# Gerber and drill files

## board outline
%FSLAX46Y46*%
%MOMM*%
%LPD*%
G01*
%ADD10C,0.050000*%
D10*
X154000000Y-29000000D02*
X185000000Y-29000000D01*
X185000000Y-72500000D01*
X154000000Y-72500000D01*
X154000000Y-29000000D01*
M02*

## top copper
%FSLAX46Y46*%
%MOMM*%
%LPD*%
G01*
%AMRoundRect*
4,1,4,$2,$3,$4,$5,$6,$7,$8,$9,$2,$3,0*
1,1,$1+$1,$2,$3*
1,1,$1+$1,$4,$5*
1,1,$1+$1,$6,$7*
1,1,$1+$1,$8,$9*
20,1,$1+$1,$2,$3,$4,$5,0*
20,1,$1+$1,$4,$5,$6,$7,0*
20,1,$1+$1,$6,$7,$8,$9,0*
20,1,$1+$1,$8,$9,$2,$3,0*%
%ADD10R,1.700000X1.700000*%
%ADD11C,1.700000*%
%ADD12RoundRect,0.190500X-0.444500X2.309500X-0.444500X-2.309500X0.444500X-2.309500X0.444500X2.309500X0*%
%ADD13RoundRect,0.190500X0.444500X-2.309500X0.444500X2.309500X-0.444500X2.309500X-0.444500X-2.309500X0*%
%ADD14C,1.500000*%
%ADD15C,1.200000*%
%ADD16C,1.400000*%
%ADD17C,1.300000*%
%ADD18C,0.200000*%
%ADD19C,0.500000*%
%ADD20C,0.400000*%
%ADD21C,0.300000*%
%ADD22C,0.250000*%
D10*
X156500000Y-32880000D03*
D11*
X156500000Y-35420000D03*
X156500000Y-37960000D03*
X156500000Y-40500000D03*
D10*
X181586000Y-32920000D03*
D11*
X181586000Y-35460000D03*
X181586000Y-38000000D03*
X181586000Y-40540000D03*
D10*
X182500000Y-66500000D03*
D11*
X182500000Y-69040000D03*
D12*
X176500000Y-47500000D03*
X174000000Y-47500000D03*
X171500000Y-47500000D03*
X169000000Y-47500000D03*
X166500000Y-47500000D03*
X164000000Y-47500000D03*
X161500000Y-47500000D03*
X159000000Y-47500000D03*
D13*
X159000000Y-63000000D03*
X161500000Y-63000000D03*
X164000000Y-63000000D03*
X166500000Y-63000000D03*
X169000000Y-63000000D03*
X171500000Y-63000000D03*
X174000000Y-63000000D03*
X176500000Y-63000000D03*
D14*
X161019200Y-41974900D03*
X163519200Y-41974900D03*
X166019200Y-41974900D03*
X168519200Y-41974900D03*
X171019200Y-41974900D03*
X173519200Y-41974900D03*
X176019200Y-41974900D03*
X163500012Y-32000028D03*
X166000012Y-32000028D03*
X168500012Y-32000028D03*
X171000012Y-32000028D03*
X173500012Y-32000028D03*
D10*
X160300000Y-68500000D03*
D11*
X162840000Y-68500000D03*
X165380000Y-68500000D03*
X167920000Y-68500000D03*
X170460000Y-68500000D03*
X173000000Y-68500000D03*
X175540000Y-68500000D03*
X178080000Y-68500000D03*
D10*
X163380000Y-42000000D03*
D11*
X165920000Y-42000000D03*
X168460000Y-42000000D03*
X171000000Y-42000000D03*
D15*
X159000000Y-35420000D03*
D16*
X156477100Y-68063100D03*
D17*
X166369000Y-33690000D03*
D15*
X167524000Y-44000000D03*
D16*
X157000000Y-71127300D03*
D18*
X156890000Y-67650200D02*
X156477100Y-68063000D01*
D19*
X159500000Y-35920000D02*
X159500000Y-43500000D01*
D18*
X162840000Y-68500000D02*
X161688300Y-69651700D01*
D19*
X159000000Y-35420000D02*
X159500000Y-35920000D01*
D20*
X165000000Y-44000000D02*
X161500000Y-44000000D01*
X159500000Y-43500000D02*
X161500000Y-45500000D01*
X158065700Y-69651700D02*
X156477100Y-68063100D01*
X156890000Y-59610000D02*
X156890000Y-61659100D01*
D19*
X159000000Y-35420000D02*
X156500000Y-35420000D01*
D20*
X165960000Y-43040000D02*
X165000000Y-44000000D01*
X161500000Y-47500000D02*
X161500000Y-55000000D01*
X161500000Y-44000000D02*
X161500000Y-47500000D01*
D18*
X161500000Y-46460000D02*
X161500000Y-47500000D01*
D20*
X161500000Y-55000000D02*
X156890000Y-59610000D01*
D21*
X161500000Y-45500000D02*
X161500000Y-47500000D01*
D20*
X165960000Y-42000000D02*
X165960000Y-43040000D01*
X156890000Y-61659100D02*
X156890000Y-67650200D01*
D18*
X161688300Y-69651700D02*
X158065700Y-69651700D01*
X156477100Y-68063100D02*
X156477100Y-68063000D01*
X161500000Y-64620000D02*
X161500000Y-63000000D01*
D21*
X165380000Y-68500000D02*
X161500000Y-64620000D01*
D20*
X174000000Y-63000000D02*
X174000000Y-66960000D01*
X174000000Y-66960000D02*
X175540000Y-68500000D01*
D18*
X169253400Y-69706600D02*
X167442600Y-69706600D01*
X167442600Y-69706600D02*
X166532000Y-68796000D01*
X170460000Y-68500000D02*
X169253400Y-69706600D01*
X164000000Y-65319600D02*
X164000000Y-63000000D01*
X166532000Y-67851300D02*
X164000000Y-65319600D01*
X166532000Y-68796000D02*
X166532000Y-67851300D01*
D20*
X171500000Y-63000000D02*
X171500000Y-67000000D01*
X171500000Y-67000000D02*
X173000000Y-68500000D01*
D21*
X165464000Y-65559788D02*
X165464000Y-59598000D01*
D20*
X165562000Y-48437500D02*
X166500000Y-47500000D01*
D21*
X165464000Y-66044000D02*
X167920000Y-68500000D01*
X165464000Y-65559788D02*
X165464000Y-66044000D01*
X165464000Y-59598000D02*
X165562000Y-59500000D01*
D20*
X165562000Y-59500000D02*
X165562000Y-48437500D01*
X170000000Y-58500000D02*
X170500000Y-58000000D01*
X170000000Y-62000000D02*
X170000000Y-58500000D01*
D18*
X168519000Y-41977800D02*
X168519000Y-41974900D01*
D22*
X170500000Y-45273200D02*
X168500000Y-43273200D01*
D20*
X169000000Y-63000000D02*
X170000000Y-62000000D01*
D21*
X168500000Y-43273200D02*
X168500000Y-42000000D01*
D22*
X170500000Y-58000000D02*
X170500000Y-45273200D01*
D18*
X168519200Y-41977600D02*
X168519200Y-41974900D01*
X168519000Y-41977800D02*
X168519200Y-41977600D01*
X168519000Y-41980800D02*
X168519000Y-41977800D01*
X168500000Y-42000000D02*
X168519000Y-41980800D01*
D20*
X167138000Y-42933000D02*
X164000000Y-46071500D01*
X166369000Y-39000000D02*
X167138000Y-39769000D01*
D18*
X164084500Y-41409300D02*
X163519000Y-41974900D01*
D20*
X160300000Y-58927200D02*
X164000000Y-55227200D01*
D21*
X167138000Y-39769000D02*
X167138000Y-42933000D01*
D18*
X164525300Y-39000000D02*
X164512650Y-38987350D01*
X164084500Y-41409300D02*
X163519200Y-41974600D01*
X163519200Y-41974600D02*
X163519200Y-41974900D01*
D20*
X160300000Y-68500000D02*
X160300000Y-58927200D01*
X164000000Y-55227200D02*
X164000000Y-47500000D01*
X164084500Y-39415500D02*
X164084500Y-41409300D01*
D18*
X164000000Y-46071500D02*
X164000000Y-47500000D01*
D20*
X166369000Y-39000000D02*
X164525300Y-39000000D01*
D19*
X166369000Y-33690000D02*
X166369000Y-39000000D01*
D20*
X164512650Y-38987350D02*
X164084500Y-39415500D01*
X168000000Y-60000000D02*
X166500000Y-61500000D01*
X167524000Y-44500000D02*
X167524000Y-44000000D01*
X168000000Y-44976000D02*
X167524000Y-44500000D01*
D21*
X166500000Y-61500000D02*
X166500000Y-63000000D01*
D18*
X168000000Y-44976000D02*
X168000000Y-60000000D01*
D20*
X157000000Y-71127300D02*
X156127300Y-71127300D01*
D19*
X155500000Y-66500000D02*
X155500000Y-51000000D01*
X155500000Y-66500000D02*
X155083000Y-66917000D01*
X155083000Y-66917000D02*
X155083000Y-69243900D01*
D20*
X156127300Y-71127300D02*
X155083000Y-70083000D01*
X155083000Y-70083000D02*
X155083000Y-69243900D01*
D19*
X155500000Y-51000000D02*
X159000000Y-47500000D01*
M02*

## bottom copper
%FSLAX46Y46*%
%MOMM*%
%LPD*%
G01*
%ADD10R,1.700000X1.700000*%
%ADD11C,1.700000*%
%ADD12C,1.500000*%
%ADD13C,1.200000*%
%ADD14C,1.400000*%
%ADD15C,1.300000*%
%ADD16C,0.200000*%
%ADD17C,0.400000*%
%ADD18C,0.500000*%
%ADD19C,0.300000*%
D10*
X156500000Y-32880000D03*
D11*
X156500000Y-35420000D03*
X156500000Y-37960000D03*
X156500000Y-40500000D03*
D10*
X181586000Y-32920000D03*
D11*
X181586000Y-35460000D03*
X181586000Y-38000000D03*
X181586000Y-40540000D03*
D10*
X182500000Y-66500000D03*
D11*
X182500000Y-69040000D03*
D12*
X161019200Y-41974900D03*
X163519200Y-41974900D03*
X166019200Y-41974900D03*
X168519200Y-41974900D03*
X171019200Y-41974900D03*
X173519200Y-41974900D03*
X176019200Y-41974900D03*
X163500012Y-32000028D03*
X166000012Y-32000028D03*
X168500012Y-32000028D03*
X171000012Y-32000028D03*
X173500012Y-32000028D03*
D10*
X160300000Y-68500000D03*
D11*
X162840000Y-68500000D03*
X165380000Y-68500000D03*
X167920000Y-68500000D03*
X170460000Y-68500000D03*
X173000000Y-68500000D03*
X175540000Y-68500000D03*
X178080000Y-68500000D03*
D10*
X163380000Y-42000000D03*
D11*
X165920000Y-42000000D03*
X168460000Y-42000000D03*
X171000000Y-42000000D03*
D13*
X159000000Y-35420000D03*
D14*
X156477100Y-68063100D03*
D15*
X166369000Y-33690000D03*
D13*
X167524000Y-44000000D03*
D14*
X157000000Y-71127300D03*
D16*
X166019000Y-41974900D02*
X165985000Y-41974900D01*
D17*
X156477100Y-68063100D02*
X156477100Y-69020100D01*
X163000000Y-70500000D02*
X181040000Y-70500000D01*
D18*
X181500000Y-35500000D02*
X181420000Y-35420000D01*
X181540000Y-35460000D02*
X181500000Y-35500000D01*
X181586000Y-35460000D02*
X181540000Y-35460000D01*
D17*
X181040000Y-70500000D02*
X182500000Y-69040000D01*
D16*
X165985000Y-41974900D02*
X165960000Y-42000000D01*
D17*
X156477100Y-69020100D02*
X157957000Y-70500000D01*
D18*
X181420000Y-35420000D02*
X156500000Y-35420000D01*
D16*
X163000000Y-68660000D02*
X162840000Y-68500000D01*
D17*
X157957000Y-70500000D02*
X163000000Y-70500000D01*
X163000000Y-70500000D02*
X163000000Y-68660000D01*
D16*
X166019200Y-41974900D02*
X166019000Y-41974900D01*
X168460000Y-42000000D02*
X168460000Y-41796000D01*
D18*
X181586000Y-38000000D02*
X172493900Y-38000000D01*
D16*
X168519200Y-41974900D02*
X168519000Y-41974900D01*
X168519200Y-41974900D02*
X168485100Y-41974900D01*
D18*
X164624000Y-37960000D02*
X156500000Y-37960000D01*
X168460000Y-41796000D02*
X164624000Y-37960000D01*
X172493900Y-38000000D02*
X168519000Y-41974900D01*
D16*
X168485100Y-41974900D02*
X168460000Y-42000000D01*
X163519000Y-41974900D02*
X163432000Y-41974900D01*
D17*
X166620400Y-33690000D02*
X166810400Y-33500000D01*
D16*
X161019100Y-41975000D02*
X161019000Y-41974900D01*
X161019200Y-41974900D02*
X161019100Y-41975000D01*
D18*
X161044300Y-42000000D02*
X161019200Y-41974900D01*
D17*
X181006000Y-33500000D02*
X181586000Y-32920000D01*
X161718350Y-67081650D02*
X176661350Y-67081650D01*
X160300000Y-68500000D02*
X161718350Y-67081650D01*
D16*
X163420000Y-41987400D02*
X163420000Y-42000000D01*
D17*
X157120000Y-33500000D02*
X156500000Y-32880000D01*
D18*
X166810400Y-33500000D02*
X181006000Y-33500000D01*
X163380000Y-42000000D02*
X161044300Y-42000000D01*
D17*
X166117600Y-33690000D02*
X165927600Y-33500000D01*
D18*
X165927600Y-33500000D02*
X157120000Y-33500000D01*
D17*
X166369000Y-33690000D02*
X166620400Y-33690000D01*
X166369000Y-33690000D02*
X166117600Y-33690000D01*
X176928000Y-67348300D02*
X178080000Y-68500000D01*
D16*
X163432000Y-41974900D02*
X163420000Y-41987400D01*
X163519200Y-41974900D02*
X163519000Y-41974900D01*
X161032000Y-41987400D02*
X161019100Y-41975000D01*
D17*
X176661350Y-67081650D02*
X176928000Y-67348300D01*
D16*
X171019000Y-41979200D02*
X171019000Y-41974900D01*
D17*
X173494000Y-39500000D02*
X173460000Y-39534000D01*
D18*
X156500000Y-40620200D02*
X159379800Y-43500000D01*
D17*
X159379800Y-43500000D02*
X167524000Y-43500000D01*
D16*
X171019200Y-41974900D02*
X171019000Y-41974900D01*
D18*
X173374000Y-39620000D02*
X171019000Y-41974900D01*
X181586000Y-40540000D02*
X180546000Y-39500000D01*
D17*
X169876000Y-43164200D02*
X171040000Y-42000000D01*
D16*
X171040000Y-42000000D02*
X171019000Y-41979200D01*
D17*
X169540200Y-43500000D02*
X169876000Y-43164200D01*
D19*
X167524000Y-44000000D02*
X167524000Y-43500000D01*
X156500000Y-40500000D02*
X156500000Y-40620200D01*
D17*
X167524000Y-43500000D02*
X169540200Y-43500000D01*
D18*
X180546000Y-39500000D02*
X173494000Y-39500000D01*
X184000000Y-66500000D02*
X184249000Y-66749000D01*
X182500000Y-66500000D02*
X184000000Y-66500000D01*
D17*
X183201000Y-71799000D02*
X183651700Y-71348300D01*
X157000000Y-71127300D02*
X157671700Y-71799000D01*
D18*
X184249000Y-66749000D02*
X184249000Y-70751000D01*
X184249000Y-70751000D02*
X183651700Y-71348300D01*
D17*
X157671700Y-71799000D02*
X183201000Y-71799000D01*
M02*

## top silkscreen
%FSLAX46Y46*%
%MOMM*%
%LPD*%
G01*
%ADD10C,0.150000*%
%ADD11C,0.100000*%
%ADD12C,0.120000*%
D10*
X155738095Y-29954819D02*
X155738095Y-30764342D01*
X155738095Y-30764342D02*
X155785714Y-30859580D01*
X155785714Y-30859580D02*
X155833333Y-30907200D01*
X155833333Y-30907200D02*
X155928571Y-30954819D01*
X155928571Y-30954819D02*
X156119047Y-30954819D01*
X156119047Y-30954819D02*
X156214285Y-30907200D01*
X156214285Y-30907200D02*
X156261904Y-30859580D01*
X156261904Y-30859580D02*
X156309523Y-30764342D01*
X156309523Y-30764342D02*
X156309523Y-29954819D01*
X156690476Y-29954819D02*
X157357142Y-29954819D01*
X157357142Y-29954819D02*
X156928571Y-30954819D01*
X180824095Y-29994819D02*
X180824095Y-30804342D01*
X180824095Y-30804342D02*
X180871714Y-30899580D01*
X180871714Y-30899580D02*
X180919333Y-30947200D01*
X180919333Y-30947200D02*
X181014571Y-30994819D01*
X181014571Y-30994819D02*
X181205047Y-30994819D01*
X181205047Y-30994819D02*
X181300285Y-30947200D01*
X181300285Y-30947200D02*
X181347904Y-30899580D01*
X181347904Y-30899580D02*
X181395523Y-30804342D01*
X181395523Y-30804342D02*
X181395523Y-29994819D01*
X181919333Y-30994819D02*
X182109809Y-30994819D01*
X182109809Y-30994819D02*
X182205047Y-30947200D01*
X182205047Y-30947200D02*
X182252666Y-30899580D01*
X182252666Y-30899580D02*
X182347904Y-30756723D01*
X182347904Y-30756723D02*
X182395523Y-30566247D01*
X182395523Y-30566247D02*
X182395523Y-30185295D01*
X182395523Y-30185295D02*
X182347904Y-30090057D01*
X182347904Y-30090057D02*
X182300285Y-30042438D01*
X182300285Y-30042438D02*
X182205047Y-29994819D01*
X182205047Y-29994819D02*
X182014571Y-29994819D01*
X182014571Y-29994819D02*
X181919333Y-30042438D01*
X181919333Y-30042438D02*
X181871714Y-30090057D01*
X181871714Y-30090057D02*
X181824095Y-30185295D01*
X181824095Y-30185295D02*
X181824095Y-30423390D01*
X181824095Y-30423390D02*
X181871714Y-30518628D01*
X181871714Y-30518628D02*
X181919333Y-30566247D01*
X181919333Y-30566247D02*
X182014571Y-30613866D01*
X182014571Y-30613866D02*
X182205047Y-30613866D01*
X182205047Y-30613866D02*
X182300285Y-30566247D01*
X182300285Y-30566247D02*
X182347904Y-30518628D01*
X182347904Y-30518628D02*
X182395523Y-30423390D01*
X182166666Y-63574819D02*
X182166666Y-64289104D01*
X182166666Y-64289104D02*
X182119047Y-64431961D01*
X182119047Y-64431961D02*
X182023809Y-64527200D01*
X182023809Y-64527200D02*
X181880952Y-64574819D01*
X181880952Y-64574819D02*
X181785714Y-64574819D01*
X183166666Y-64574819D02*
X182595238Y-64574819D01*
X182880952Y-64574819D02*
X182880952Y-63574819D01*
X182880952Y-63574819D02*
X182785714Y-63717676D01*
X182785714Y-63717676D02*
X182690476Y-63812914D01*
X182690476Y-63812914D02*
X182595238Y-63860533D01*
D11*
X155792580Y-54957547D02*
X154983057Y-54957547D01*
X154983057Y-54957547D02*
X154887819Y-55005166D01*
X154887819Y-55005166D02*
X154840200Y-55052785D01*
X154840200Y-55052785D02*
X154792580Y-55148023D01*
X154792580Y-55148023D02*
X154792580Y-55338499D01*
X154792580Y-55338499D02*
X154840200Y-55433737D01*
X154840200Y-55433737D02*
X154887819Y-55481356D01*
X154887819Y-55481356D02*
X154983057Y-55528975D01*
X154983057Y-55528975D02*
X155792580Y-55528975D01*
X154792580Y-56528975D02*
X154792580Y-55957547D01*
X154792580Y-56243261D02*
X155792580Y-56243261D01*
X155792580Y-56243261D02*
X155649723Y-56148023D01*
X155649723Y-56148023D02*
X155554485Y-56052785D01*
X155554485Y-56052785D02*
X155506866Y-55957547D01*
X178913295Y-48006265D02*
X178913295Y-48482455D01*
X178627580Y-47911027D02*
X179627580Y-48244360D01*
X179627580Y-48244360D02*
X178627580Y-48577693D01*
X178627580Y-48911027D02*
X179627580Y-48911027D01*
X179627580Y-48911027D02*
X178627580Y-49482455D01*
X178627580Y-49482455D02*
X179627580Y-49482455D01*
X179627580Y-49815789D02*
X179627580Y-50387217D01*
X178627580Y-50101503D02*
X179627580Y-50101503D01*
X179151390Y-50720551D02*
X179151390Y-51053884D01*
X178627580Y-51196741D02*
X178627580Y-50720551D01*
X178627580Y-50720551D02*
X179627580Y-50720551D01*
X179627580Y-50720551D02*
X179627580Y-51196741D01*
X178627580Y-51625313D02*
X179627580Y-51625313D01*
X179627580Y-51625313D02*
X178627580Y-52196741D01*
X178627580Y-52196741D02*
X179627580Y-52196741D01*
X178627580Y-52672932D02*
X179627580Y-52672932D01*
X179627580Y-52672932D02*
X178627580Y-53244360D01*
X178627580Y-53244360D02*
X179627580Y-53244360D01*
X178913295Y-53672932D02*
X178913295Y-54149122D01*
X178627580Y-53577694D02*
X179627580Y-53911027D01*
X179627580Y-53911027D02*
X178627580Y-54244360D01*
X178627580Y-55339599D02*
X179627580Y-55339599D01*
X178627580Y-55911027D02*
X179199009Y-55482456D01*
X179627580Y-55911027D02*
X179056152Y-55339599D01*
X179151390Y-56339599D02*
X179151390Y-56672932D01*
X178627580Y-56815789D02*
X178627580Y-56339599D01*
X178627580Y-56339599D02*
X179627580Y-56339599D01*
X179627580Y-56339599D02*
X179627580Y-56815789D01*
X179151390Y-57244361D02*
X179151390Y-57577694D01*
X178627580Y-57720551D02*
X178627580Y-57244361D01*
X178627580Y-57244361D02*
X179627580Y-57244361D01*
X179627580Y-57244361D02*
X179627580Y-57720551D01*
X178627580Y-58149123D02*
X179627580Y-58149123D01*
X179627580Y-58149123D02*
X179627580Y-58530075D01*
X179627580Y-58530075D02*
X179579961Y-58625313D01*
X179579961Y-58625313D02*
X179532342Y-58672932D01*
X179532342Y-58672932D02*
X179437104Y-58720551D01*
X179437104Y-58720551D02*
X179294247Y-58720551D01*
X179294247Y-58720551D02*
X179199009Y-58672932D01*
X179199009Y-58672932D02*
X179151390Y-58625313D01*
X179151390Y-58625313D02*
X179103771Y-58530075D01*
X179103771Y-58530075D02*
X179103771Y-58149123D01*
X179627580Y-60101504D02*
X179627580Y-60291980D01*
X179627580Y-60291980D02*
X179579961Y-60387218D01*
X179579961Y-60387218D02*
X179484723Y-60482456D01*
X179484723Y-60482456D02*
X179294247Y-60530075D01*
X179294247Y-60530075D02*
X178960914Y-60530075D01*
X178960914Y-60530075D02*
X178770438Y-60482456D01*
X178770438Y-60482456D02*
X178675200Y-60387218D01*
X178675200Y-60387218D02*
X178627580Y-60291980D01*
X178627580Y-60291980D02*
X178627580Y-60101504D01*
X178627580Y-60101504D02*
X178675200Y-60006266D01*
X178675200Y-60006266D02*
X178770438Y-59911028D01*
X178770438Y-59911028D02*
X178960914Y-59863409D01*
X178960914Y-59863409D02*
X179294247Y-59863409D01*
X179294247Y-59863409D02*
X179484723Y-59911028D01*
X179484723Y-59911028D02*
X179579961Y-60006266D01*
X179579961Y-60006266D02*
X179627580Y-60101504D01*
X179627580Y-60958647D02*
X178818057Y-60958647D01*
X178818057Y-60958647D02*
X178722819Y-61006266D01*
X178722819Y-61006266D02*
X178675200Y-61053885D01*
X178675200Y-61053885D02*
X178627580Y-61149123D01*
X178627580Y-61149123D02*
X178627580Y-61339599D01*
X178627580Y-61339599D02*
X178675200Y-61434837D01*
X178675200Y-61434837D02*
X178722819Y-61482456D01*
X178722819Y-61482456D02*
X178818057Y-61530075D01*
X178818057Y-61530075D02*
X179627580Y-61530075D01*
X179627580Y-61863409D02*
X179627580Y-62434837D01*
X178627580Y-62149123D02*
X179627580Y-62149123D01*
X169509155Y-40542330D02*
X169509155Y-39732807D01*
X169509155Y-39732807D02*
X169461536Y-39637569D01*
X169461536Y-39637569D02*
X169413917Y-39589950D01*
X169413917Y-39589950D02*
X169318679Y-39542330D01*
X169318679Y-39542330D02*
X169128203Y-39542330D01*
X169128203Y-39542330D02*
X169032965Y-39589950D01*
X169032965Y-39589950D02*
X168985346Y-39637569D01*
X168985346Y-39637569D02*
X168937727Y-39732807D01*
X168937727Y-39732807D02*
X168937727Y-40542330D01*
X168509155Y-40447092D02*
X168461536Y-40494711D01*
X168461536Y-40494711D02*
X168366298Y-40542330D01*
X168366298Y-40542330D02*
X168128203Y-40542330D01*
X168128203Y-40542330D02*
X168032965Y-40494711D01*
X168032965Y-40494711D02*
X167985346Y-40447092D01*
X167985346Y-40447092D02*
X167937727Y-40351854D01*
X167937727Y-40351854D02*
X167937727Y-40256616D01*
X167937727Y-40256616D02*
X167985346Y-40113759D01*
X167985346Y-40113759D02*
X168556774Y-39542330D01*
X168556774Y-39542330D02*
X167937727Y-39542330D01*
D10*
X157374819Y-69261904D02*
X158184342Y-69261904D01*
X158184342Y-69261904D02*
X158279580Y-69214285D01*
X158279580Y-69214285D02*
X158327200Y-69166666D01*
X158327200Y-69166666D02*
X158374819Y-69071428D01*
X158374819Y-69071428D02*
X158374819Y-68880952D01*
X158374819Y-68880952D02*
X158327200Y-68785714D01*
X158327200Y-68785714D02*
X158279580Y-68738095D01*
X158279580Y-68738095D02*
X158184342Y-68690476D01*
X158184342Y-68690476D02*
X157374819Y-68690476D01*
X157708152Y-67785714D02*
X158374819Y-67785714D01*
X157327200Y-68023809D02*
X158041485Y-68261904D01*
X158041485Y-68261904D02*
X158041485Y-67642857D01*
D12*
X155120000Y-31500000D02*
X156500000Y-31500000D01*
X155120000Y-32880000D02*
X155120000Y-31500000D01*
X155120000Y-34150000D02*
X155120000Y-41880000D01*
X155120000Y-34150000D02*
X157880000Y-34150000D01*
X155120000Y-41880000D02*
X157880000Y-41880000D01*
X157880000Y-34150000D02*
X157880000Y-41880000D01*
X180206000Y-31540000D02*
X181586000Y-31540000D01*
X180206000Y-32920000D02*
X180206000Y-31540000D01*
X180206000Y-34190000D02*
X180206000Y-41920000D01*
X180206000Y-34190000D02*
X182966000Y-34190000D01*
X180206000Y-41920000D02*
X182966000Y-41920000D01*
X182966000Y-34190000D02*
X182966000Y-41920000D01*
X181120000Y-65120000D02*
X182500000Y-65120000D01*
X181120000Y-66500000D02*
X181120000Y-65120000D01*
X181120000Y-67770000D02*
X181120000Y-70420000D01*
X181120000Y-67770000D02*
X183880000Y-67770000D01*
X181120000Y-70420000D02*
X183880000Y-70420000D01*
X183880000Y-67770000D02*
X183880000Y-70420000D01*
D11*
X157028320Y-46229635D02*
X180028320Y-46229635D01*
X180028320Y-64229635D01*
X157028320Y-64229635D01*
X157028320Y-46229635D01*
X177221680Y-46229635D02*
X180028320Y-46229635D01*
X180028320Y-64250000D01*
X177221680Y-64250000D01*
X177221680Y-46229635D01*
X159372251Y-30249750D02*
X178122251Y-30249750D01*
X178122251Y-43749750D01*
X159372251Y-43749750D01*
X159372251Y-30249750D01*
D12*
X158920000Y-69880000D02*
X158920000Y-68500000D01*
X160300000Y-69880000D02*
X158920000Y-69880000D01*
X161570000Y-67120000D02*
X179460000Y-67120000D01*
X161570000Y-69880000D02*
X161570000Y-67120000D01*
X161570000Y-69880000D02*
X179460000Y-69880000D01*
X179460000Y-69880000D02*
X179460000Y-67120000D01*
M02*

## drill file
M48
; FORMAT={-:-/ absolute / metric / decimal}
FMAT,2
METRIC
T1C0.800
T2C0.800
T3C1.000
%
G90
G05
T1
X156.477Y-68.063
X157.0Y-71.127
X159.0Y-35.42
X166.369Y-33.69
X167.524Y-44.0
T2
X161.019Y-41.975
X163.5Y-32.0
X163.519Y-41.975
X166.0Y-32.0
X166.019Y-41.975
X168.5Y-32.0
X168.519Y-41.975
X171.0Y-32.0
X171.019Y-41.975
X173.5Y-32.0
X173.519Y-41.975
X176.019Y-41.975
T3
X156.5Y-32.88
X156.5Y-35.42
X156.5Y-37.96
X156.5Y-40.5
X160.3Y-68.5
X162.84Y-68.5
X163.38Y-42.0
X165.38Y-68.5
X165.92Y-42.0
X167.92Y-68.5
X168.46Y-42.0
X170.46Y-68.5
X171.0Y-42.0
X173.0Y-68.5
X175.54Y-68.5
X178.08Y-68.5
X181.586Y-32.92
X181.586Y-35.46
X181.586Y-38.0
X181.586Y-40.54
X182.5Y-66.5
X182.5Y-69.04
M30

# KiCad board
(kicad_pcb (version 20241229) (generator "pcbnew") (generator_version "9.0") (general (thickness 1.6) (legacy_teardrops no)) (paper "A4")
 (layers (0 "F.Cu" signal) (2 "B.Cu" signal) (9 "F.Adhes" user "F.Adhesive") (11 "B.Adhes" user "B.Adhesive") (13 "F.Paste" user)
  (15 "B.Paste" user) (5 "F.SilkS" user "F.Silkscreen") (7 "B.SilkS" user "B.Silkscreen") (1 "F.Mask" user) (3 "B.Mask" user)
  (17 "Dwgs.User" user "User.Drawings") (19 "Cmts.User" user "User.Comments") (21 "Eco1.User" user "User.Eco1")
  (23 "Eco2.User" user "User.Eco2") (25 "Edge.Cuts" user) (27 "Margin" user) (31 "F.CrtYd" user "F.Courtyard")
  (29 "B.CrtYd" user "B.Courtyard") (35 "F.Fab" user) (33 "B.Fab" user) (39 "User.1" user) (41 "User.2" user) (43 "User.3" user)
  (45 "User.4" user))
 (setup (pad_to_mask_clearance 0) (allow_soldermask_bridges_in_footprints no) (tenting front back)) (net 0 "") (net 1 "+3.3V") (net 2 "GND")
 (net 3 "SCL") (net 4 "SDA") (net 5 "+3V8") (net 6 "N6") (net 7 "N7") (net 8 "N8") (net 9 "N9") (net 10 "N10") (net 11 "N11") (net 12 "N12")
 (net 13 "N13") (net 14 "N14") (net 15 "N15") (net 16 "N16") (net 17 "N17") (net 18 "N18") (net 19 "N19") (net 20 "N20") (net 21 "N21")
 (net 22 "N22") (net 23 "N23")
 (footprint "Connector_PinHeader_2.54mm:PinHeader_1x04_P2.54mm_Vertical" (layer "F.Cu") (at 156.5 32.88)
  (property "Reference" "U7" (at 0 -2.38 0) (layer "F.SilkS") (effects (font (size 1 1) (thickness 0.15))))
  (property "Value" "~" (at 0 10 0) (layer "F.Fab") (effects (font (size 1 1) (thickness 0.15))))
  (fp_line (start -1.38 -1.38) (end 0 -1.38) (stroke (width 0.12) (type solid)) (layer "F.SilkS"))
  (fp_line (start -1.38 0) (end -1.38 -1.38) (stroke (width 0.12) (type solid)) (layer "F.SilkS"))
  (fp_line (start -1.38 1.27) (end -1.38 9) (stroke (width 0.12) (type solid)) (layer "F.SilkS"))
  (fp_line (start -1.38 1.27) (end 1.38 1.27) (stroke (width 0.12) (type solid)) (layer "F.SilkS"))
  (fp_line (start -1.38 9) (end 1.38 9) (stroke (width 0.12) (type solid)) (layer "F.SilkS"))
  (fp_line (start 1.38 1.27) (end 1.38 9) (stroke (width 0.12) (type solid)) (layer "F.SilkS"))
  (pad "1" thru_hole rect (at 0 0) (size 1.7 1.7) (drill 1) (layers "*.Cu" "*.Mask") (remove_unused_layers no) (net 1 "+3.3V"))
  (pad "2" thru_hole circle (at 0 2.54) (size 1.7 1.7) (drill 1) (layers "*.Cu" "*.Mask") (remove_unused_layers no) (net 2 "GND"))
  (pad "3" thru_hole circle (at 0 5.08) (size 1.7 1.7) (drill 1) (layers "*.Cu" "*.Mask") (remove_unused_layers no) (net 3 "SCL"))
  (pad "4" thru_hole circle (at 0 7.62) (size 1.7 1.7) (drill 1) (layers "*.Cu" "*.Mask") (remove_unused_layers no) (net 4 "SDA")))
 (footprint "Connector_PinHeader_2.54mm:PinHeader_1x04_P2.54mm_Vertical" (layer "F.Cu") (at 181.586 32.92)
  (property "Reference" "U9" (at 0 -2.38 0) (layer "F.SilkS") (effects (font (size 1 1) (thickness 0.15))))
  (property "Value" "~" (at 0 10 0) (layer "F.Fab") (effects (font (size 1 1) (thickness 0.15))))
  (fp_line (start -1.38 -1.38) (end 0 -1.38) (stroke (width 0.12) (type solid)) (layer "F.SilkS"))
  (fp_line (start -1.38 0) (end -1.38 -1.38) (stroke (width 0.12) (type solid)) (layer "F.SilkS"))
  (fp_line (start -1.38 1.27) (end -1.38 9) (stroke (width 0.12) (type solid)) (layer "F.SilkS"))
  (fp_line (start -1.38 1.27) (end 1.38 1.27) (stroke (width 0.12) (type solid)) (layer "F.SilkS"))
  (fp_line (start -1.38 9) (end 1.38 9) (stroke (width 0.12) (type solid)) (layer "F.SilkS"))
  (fp_line (start 1.38 1.27) (end 1.38 9) (stroke (width 0.12) (type solid)) (layer "F.SilkS"))
  (pad "1" thru_hole rect (at 0 0) (size 1.7 1.7) (drill 1) (layers "*.Cu" "*.Mask") (remove_unused_layers no) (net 1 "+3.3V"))
  (pad "2" thru_hole circle (at 0 2.54) (size 1.7 1.7) (drill 1) (layers "*.Cu" "*.Mask") (remove_unused_layers no) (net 2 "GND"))
  (pad "3" thru_hole circle (at 0 5.08) (size 1.7 1.7) (drill 1) (layers "*.Cu" "*.Mask") (remove_unused_layers no) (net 3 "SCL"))
  (pad "4" thru_hole circle (at 0 7.62) (size 1.7 1.7) (drill 1) (layers "*.Cu" "*.Mask") (remove_unused_layers no) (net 4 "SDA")))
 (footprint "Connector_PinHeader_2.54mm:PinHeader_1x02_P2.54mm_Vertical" (layer "F.Cu") (at 182.5 66.5)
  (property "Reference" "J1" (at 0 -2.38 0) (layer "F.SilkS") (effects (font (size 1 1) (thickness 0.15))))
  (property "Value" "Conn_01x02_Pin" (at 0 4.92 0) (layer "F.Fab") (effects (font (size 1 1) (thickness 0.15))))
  (fp_line (start -1.38 -1.38) (end 0 -1.38) (stroke (width 0.12) (type solid)) (layer "F.SilkS"))
  (fp_line (start -1.38 0) (end -1.38 -1.38) (stroke (width 0.12) (type solid)) (layer "F.SilkS"))
  (fp_line (start -1.38 1.27) (end -1.38 3.92) (stroke (width 0.12) (type solid)) (layer "F.SilkS"))
  (fp_line (start -1.38 1.27) (end 1.38 1.27) (stroke (width 0.12) (type solid)) (layer "F.SilkS"))
  (fp_line (start -1.38 3.92) (end 1.38 3.92) (stroke (width 0.12) (type solid)) (layer "F.SilkS"))
  (fp_line (start 1.38 1.27) (end 1.38 3.92) (stroke (width 0.12) (type solid)) (layer "F.SilkS"))
  (pad "1" thru_hole rect (at 0 0) (size 1.7 1.7) (drill 1) (layers "*.Cu" "*.Mask") (remove_unused_layers no) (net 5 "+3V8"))
  (pad "2" thru_hole circle (at 0 2.54) (size 1.7 1.7) (drill 1) (layers "*.Cu" "*.Mask") (remove_unused_layers no) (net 2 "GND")))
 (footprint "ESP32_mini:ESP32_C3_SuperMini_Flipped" (layer "F.Cu") (at 176.5 47.5 -90)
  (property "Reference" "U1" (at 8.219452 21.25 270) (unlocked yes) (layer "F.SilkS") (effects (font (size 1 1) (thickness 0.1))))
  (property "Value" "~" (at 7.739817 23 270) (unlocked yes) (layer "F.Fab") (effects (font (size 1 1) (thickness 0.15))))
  (fp_rect (start -1.270365 -3.52832) (end 16.729635 19.47168) (stroke (width 0.1) (type default)) (fill no) (layer "F.SilkS"))
  (fp_rect (start -1.270365 -3.52832) (end 16.75 -0.72168) (stroke (width 0.1) (type default)) (fill no) (layer "F.SilkS"))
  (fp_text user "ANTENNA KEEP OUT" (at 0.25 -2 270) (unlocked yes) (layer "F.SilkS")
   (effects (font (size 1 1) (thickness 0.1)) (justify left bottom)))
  (pad "0" smd roundrect (at 0 0 270) (size 5 1.27) (layers "F.Cu" "F.Mask" "F.Paste") (roundrect_rratio 0.15) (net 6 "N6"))
  (pad "1" smd roundrect (at 0 2.5 270) (size 5 1.27) (layers "F.Cu" "F.Mask" "F.Paste") (roundrect_rratio 0.15) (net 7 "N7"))
  (pad "2" smd roundrect (at 0 5 270) (size 5 1.27) (layers "F.Cu" "F.Mask" "F.Paste") (roundrect_rratio 0.15) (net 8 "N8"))
  (pad "3" smd roundrect (at 0 7.5 270) (size 5 1.27) (layers "F.Cu" "F.Mask" "F.Paste") (roundrect_rratio 0.15) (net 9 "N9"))
  (pad "4" smd roundrect (at 0 10 270) (size 5 1.27) (layers "F.Cu" "F.Mask" "F.Paste") (roundrect_rratio 0.15) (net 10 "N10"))
  (pad "5" smd roundrect (at 0 12.5 270) (size 5 1.27) (layers "F.Cu" "F.Mask" "F.Paste") (roundrect_rratio 0.15) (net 1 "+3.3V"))
  (pad "6" smd roundrect (at 0 15 270) (size 5 1.27) (layers "F.Cu" "F.Mask" "F.Paste") (roundrect_rratio 0.15) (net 2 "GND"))
  (pad "7" smd roundrect (at 0 17.5 270) (size 5 1.27) (layers "F.Cu" "F.Mask" "F.Paste") (roundrect_rratio 0.15) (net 5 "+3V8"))
  (pad "8" smd roundrect (at 15.5 17.5 90) (size 5 1.27) (layers "F.Cu" "F.Mask" "F.Paste") (roundrect_rratio 0.15) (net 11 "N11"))
  (pad "9" smd roundrect (at 15.5 15 90) (size 5 1.27) (layers "F.Cu" "F.Mask" "F.Paste") (roundrect_rratio 0.15) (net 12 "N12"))
  (pad "10" smd roundrect (at 15.5 12.5 90) (size 5 1.27) (layers "F.Cu" "F.Mask" "F.Paste") (roundrect_rratio 0.15) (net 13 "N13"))
  (pad "11" smd roundrect (at 15.5 10 90) (size 5 1.27) (layers "F.Cu" "F.Mask" "F.Paste") (roundrect_rratio 0.15) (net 4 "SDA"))
  (pad "12" smd roundrect (at 15.5 7.5 90) (size 5 1.27) (layers "F.Cu" "F.Mask" "F.Paste") (roundrect_rratio 0.15) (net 3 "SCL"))
  (pad "13" smd roundrect (at 15.5 5 90) (size 5 1.27) (layers "F.Cu" "F.Mask" "F.Paste") (roundrect_rratio 0.15) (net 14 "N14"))
  (pad "14" smd roundrect (at 15.5 2.5 90) (size 5 1.27) (layers "F.Cu" "F.Mask" "F.Paste") (roundrect_rratio 0.15) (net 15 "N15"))
  (pad "15" smd roundrect (at 15.5 0 90) (size 5 1.27) (layers "F.Cu" "F.Mask" "F.Paste") (roundrect_rratio 0.15) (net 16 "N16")))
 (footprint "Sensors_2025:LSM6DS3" (layer "F.Cu") (at 161.0192 41.9749 90)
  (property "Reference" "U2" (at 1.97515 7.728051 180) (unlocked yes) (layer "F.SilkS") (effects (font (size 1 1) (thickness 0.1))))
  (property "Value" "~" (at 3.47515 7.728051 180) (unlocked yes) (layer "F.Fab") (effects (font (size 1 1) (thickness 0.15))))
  (fp_rect (start -1.77485 -1.646949) (end 11.72515 17.103051) (stroke (width 0.1) (type default)) (fill no) (layer "F.SilkS"))
  (pad "0" thru_hole circle (at 0 0 90) (size 1.5 1.5) (drill 0.8) (layers "*.Cu" "*.Mask") (remove_unused_layers no) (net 1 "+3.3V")
   (thermal_bridge_angle 90))
  (pad "1" thru_hole circle (at 0 2.5 90) (size 1.5 1.5) (drill 0.8) (layers "*.Cu" "*.Mask") (remove_unused_layers no) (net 1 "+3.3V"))
  (pad "2" thru_hole circle (at 0 5 90) (size 1.5 1.5) (drill 0.8) (layers "*.Cu" "*.Mask") (remove_unused_layers no) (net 2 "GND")
   (thermal_bridge_angle 90))
  (pad "3" thru_hole circle (at 0 7.5 90) (size 1.5 1.5) (drill 0.8) (layers "*.Cu" "*.Mask") (remove_unused_layers no) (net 3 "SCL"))
  (pad "4" thru_hole circle (at 0 10 90) (size 1.5 1.5) (drill 0.8) (layers "*.Cu" "*.Mask") (remove_unused_layers no) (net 4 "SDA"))
  (pad "5" thru_hole circle (at 0 12.5 90) (size 1.5 1.5) (drill 0.8) (layers "*.Cu" "*.Mask") (remove_unused_layers no) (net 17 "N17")
   (thermal_bridge_angle 90))
  (pad "6" thru_hole circle (at 0 15 90) (size 1.5 1.5) (drill 0.8) (layers "*.Cu" "*.Mask") (remove_unused_layers no) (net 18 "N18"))
  (pad "7" thru_hole circle (at 9.974872 2.480812 90) (size 1.5 1.5) (drill 0.8) (layers "*.Cu" "*.Mask") (remove_unused_layers no)
   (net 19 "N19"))
  (pad "8" thru_hole circle (at 9.974872 4.980812 90) (size 1.5 1.5) (drill 0.8) (layers "*.Cu" "*.Mask") (remove_unused_layers no)
   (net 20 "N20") (thermal_bridge_angle 90))
  (pad "9" thru_hole circle (at 9.974872 7.480812 90) (size 1.5 1.5) (drill 0.8) (layers "*.Cu" "*.Mask") (remove_unused_layers no)
   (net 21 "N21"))
  (pad "10" thru_hole circle (at 9.974872 9.980812 90) (size 1.5 1.5) (drill 0.8) (layers "*.Cu" "*.Mask") (remove_unused_layers no)
   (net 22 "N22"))
  (pad "11" thru_hole circle (at 9.974872 12.480812 90) (size 1.5 1.5) (drill 0.8) (layers "*.Cu" "*.Mask") (remove_unused_layers no)
   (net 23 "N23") (thermal_bridge_angle 90)))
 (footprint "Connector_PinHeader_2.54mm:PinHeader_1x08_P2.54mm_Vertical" (layer "F.Cu") (at 160.3 68.5 90)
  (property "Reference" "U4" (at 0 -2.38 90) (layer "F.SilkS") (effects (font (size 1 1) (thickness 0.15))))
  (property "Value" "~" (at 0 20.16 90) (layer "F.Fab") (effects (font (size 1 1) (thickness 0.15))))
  (fp_line (start -1.38 -1.38) (end 0 -1.38) (stroke (width 0.12) (type solid)) (layer "F.SilkS"))
  (fp_line (start -1.38 0) (end -1.38 -1.38) (stroke (width 0.12) (type solid)) (layer "F.SilkS"))
  (fp_line (start 1.38 1.27) (end 1.38 19.16) (stroke (width 0.12) (type solid)) (layer "F.SilkS"))
  (fp_line (start -1.38 1.27) (end 1.38 1.27) (stroke (width 0.12) (type solid)) (layer "F.SilkS"))
  (fp_line (start -1.38 1.27) (end -1.38 19.16) (stroke (width 0.12) (type solid)) (layer "F.SilkS"))
  (fp_line (start -1.38 19.16) (end 1.38 19.16) (stroke (width 0.12) (type solid)) (layer "F.SilkS"))
  (pad "1" thru_hole rect (at 0 0 90) (size 1.7 1.7) (drill 1) (layers "*.Cu" "*.Mask") (remove_unused_layers no) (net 1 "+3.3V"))
  (pad "2" thru_hole circle (at 0 2.54 90) (size 1.7 1.7) (drill 1) (layers "*.Cu" "*.Mask") (remove_unused_layers no) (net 2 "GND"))
  (pad "3" thru_hole circle (at 0 5.08 90) (size 1.7 1.7) (drill 1) (layers "*.Cu" "*.Mask") (remove_unused_layers no) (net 12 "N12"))
  (pad "4" thru_hole circle (at 0 7.62 90) (size 1.7 1.7) (drill 1) (layers "*.Cu" "*.Mask") (remove_unused_layers no) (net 10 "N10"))
  (pad "5" thru_hole circle (at 0 10.16 90) (size 1.7 1.7) (drill 1) (layers "*.Cu" "*.Mask") (remove_unused_layers no) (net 13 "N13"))
  (pad "6" thru_hole circle (at 0 12.7 90) (size 1.7 1.7) (drill 1) (layers "*.Cu" "*.Mask") (remove_unused_layers no) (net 14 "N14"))
  (pad "7" thru_hole circle (at 0 15.24 90) (size 1.7 1.7) (drill 1) (layers "*.Cu" "*.Mask") (remove_unused_layers no) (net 15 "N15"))
  (pad "8" thru_hole circle (at 0 17.78 90) (size 1.7 1.7) (drill 1) (layers "*.Cu" "*.Mask") (remove_unused_layers no) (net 1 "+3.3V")))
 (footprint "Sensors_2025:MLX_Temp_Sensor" (layer "B.Cu") (at 163.38 42 -90)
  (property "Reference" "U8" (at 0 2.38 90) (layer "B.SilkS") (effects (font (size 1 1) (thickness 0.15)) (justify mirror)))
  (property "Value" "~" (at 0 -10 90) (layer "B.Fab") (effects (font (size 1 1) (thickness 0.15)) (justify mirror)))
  (pad "1" thru_hole rect (at 0 0 270) (size 1.7 1.7) (drill 1) (layers "*.Cu" "*.Mask") (remove_unused_layers no) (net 1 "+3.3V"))
  (pad "2" thru_hole circle (at 0 -2.54 270) (size 1.7 1.7) (drill 1) (layers "*.Cu" "*.Mask") (remove_unused_layers no) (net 2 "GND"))
  (pad "3" thru_hole circle (at 0 -5.08 270) (size 1.7 1.7) (drill 1) (layers "*.Cu" "*.Mask") (remove_unused_layers no) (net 3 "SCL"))
  (pad "4" thru_hole circle (at 0 -7.62 270) (size 1.7 1.7) (drill 1) (layers "*.Cu" "*.Mask") (remove_unused_layers no) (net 4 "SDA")))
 (gr_rect (start 154 29) (end 185 72.5) (stroke (width 0.05) (type default)) (fill no) (layer "Edge.Cuts"))
 (segment (start 156.89 67.6502) (end 156.4771 68.063) (width 0.2) (layer "F.Cu") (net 2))
 (segment (start 159.5 35.92) (end 159.5 43.5) (width 0.5) (layer "F.Cu") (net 2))
 (segment (start 162.84 68.5) (end 161.6883 69.6517) (width 0.2) (layer "F.Cu") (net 2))
 (segment (start 159 35.42) (end 159.5 35.92) (width 0.5) (layer "F.Cu") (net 2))
 (segment (start 165 44) (end 161.5 44) (width 0.4) (layer "F.Cu") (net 2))
 (segment (start 159.5 43.5) (end 161.5 45.5) (width 0.4) (layer "F.Cu") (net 2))
 (segment (start 158.0657 69.6517) (end 156.4771 68.0631) (width 0.4) (layer "F.Cu") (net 2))
 (segment (start 156.89 59.61) (end 156.89 61.6591) (width 0.4) (layer "F.Cu") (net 2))
 (segment (start 159 35.42) (end 156.5 35.42) (width 0.5) (layer "F.Cu") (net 2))
 (segment (start 165.96 43.04) (end 165 44) (width 0.4) (layer "F.Cu") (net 2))
 (segment (start 161.5 47.5) (end 161.5 55) (width 0.4) (layer "F.Cu") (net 2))
 (segment (start 161.5 44) (end 161.5 47.5) (width 0.4) (layer "F.Cu") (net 2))
 (segment (start 161.5 46.46) (end 161.5 47.5) (width 0.2) (layer "F.Cu") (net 2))
 (segment (start 161.5 55) (end 156.89 59.61) (width 0.4) (layer "F.Cu") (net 2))
 (segment (start 161.5 45.5) (end 161.5 47.5) (width 0.3) (layer "F.Cu") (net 2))
 (segment (start 165.96 42) (end 165.96 43.04) (width 0.4) (layer "F.Cu") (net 2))
 (segment (start 156.89 61.6591) (end 156.89 67.6502) (width 0.4) (layer "F.Cu") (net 2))
 (segment (start 161.6883 69.6517) (end 158.0657 69.6517) (width 0.2) (layer "F.Cu") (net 2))
 (segment (start 156.4771 68.0631) (end 156.4771 68.063) (width 0.2) (layer "F.Cu") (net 2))
 (via (at 159 35.42) (size 1.2) (drill 0.8) (layers "F.Cu" "B.Cu") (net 2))
 (via (at 156.4771 68.0631) (size 1.4) (drill 0.8) (layers "F.Cu" "B.Cu") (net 2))
 (segment (start 166.019 41.9749) (end 165.985 41.9749) (width 0.2) (layer "B.Cu") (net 2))
 (segment (start 156.4771 68.0631) (end 156.4771 69.0201) (width 0.4) (layer "B.Cu") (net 2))
 (segment (start 163 70.5) (end 181.04 70.5) (width 0.4) (layer "B.Cu") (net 2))
 (segment (start 181.5 35.5) (end 181.42 35.42) (width 0.5) (layer "B.Cu") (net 2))
 (segment (start 181.54 35.46) (end 181.5 35.5) (width 0.5) (layer "B.Cu") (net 2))
 (segment (start 181.586 35.46) (end 181.54 35.46) (width 0.5) (layer "B.Cu") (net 2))
 (segment (start 181.04 70.5) (end 182.5 69.04) (width 0.4) (layer "B.Cu") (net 2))
 (segment (start 165.985 41.9749) (end 165.96 42) (width 0.2) (layer "B.Cu") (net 2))
 (segment (start 156.4771 69.0201) (end 157.957 70.5) (width 0.4) (layer "B.Cu") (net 2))
 (segment (start 181.42 35.42) (end 156.5 35.42) (width 0.5) (layer "B.Cu") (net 2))
 (segment (start 163 68.66) (end 162.84 68.5) (width 0.2) (layer "B.Cu") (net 2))
 (segment (start 157.957 70.5) (end 163 70.5) (width 0.4) (layer "B.Cu") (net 2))
 (segment (start 163 70.5) (end 163 68.66) (width 0.4) (layer "B.Cu") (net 2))
 (segment (start 166.0192 41.9749) (end 166.019 41.9749) (width 0.2) (layer "B.Cu") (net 2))
 (segment (start 161.5 64.62) (end 161.5 63) (width 0.2) (layer "F.Cu") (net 12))
 (segment (start 165.38 68.5) (end 161.5 64.62) (width 0.3) (layer "F.Cu") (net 12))
 (segment (start 174 63) (end 174 66.96) (width 0.4) (layer "F.Cu") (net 15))
 (segment (start 174 66.96) (end 175.54 68.5) (width 0.4) (layer "F.Cu") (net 15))
 (segment (start 169.2534 69.7066) (end 167.4426 69.7066) (width 0.2) (layer "F.Cu") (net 13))
 (segment (start 167.4426 69.7066) (end 166.532 68.796) (width 0.2) (layer "F.Cu") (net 13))
 (segment (start 170.46 68.5) (end 169.2534 69.7066) (width 0.2) (layer "F.Cu") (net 13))
 (segment (start 164 65.3196) (end 164 63) (width 0.2) (layer "F.Cu") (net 13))
 (segment (start 166.532 67.8513) (end 164 65.3196) (width 0.2) (layer "F.Cu") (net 13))
 (segment (start 166.532 68.796) (end 166.532 67.8513) (width 0.2) (layer "F.Cu") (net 13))
 (segment (start 171.5 63) (end 171.5 67) (width 0.4) (layer "F.Cu") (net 14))
 (segment (start 171.5 67) (end 173 68.5) (width 0.4) (layer "F.Cu") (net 14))
 (segment (start 165.464 65.559788) (end 165.464 59.598) (width 0.3) (layer "F.Cu") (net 10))
 (segment (start 165.562 48.4375) (end 166.5 47.5) (width 0.4) (layer "F.Cu") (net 10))
 (segment (start 165.464 66.044) (end 167.92 68.5) (width 0.3) (layer "F.Cu") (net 10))
 (segment (start 165.464 65.559788) (end 165.464 66.044) (width 0.3) (layer "F.Cu") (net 10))
 (segment (start 165.464 59.598) (end 165.562 59.5) (width 0.3) (layer "F.Cu") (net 10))
 (segment (start 165.562 59.5) (end 165.562 48.4375) (width 0.4) (layer "F.Cu") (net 10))
 (segment (start 170 58.5) (end 170.5 58) (width 0.4) (layer "F.Cu") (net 3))
 (segment (start 170 62) (end 170 58.5) (width 0.4) (layer "F.Cu") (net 3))
 (segment (start 168.519 41.9778) (end 168.519 41.9749) (width 0.2) (layer "F.Cu") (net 3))
 (segment (start 170.5 45.2732) (end 168.5 43.2732) (width 0.25) (layer "F.Cu") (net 3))
 (segment (start 169 63) (end 170 62) (width 0.4) (layer "F.Cu") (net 3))
 (segment (start 168.5 43.2732) (end 168.5 42) (width 0.3) (layer "F.Cu") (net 3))
 (segment (start 170.5 58) (end 170.5 45.2732) (width 0.25) (layer "F.Cu") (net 3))
 (segment (start 168.5192 41.9776) (end 168.5192 41.9749) (width 0.2) (layer "F.Cu") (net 3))
 (segment (start 168.519 41.9778) (end 168.5192 41.9776) (width 0.2) (layer "F.Cu") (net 3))
 (segment (start 168.519 41.9808) (end 168.519 41.9778) (width 0.2) (layer "F.Cu") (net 3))
 (segment (start 168.5 42) (end 168.519 41.9808) (width 0.2) (layer "F.Cu") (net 3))
 (segment (start 168.46 42) (end 168.46 41.796) (width 0.2) (layer "B.Cu") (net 3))
 (segment (start 181.586 38) (end 172.4939 38) (width 0.5) (layer "B.Cu") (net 3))
 (segment (start 168.5192 41.9749) (end 168.519 41.9749) (width 0.2) (layer "B.Cu") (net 3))
 (segment (start 168.5192 41.9749) (end 168.4851 41.9749) (width 0.2) (layer "B.Cu") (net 3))
 (segment (start 164.624 37.96) (end 156.5 37.96) (width 0.5) (layer "B.Cu") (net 3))
 (segment (start 168.46 41.796) (end 164.624 37.96) (width 0.5) (layer "B.Cu") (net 3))
 (segment (start 172.4939 38) (end 168.519 41.9749) (width 0.5) (layer "B.Cu") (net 3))
 (segment (start 168.4851 41.9749) (end 168.46 42) (width 0.2) (layer "B.Cu") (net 3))
 (segment (start 167.138 42.933) (end 164 46.0715) (width 0.4) (layer "F.Cu") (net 1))
 (segment (start 166.369 39) (end 167.138 39.769) (width 0.4) (layer "F.Cu") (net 1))
 (segment (start 164.0845 41.4093) (end 163.519 41.9749) (width 0.2) (layer "F.Cu") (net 1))
 (segment (start 160.3 58.9272) (end 164 55.2272) (width 0.4) (layer "F.Cu") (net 1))
 (segment (start 167.138 39.769) (end 167.138 42.933) (width 0.3) (layer "F.Cu") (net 1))
 (segment (start 164.5253 39) (end 164.51265 38.98735) (width 0.2) (layer "F.Cu") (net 1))
 (segment (start 164.0845 41.4093) (end 163.5192 41.9746) (width 0.2) (layer "F.Cu") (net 1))
 (segment (start 163.5192 41.9746) (end 163.5192 41.9749) (width 0.2) (layer "F.Cu") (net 1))
 (segment (start 160.3 68.5) (end 160.3 58.9272) (width 0.4) (layer "F.Cu") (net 1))
 (segment (start 164 55.2272) (end 164 47.5) (width 0.4) (layer "F.Cu") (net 1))
 (segment (start 164.0845 39.4155) (end 164.0845 41.4093) (width 0.4) (layer "F.Cu") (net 1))
 (segment (start 164 46.0715) (end 164 47.5) (width 0.2) (layer "F.Cu") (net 1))
 (segment (start 166.369 39) (end 164.5253 39) (width 0.4) (layer "F.Cu") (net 1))
 (segment (start 166.369 33.69) (end 166.369 39) (width 0.5) (layer "F.Cu") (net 1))
 (segment (start 164.51265 38.98735) (end 164.0845 39.4155) (width 0.4) (layer "F.Cu") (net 1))
 (via (at 166.369 33.69) (size 1.3) (drill 0.8) (layers "F.Cu" "B.Cu") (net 1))
 (segment (start 163.519 41.9749) (end 163.432 41.9749) (width 0.2) (layer "B.Cu") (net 1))
 (segment (start 166.6204 33.69) (end 166.8104 33.5) (width 0.4) (layer "B.Cu") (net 1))
 (segment (start 161.0191 41.975) (end 161.019 41.9749) (width 0.2) (layer "B.Cu") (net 1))
 (segment (start 161.0192 41.9749) (end 161.0191 41.975) (width 0.2) (layer "B.Cu") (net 1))
 (segment (start 161.0443 42) (end 161.0192 41.9749) (width 0.5) (layer "B.Cu") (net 1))
 (segment (start 181.006 33.5) (end 181.586 32.92) (width 0.4) (layer "B.Cu") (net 1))
 (segment (start 161.71835 67.08165) (end 176.66135 67.08165) (width 0.4) (layer "B.Cu") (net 1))
 (segment (start 160.3 68.5) (end 161.71835 67.08165) (width 0.4) (layer "B.Cu") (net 1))
 (segment (start 163.42 41.9874) (end 163.42 42) (width 0.2) (layer "B.Cu") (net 1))
 (segment (start 157.12 33.5) (end 156.5 32.88) (width 0.4) (layer "B.Cu") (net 1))
 (segment (start 166.8104 33.5) (end 181.006 33.5) (width 0.5) (layer "B.Cu") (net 1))
 (segment (start 163.38 42) (end 161.0443 42) (width 0.5) (layer "B.Cu") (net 1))
 (segment (start 166.1176 33.69) (end 165.9276 33.5) (width 0.4) (layer "B.Cu") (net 1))
 (segment (start 165.9276 33.5) (end 157.12 33.5) (width 0.5) (layer "B.Cu") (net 1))
 (segment (start 166.369 33.69) (end 166.6204 33.69) (width 0.4) (layer "B.Cu") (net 1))
 (segment (start 166.369 33.69) (end 166.1176 33.69) (width 0.4) (layer "B.Cu") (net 1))
 (segment (start 176.928 67.3483) (end 178.08 68.5) (width 0.4) (layer "B.Cu") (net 1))
 (segment (start 163.432 41.9749) (end 163.42 41.9874) (width 0.2) (layer "B.Cu") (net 1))
 (segment (start 163.5192 41.9749) (end 163.519 41.9749) (width 0.2) (layer "B.Cu") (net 1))
 (segment (start 161.032 41.9874) (end 161.0191 41.975) (width 0.2) (layer "B.Cu") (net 1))
 (segment (start 176.66135 67.08165) (end 176.928 67.3483) (width 0.4) (layer "B.Cu") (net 1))
 (segment (start 168 60) (end 166.5 61.5) (width 0.4) (layer "F.Cu") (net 4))
 (segment (start 167.524 44.5) (end 167.524 44) (width 0.4) (layer "F.Cu") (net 4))
 (segment (start 168 44.976) (end 167.524 44.5) (width 0.4) (layer "F.Cu") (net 4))
 (segment (start 166.5 61.5) (end 166.5 63) (width 0.3) (layer "F.Cu") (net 4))
 (segment (start 168 44.976) (end 168 60) (width 0.2) (layer "F.Cu") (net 4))
 (via (at 167.524 44) (size 1.2) (drill 0.8) (layers "F.Cu" "B.Cu") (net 4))
 (segment (start 171.019 41.9792) (end 171.019 41.9749) (width 0.2) (layer "B.Cu") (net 4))
 (segment (start 173.494 39.5) (end 173.46 39.534) (width 0.4) (layer "B.Cu") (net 4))
 (segment (start 156.5 40.6202) (end 159.3798 43.5) (width 0.5) (layer "B.Cu") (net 4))
 (segment (start 159.3798 43.5) (end 167.524 43.5) (width 0.4) (layer "B.Cu") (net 4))
 (segment (start 171.0192 41.9749) (end 171.019 41.9749) (width 0.2) (layer "B.Cu") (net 4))
 (segment (start 173.374 39.62) (end 171.019 41.9749) (width 0.5) (layer "B.Cu") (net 4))
 (segment (start 181.586 40.54) (end 180.546 39.5) (width 0.5) (layer "B.Cu") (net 4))
 (segment (start 169.876 43.1642) (end 171.04 42) (width 0.4) (layer "B.Cu") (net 4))
 (segment (start 171.04 42) (end 171.019 41.9792) (width 0.2) (layer "B.Cu") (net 4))
 (segment (start 169.5402 43.5) (end 169.876 43.1642) (width 0.4) (layer "B.Cu") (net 4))
 (segment (start 167.524 44) (end 167.524 43.5) (width 0.3) (layer "B.Cu") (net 4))
 (segment (start 156.5 40.5) (end 156.5 40.6202) (width 0.3) (layer "B.Cu") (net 4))
 (segment (start 167.524 43.5) (end 169.5402 43.5) (width 0.4) (layer "B.Cu") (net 4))
 (segment (start 180.546 39.5) (end 173.494 39.5) (width 0.5) (layer "B.Cu") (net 4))
 (segment (start 157 71.1273) (end 156.1273 71.1273) (width 0.4) (layer "F.Cu") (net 5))
 (segment (start 155.5 66.5) (end 155.5 51) (width 0.5) (layer "F.Cu") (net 5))
 (segment (start 155.5 66.5) (end 155.083 66.917) (width 0.5) (layer "F.Cu") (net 5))
 (segment (start 155.083 66.917) (end 155.083 69.2439) (width 0.5) (layer "F.Cu") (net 5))
 (segment (start 156.1273 71.1273) (end 155.083 70.083) (width 0.4) (layer "F.Cu") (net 5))
 (segment (start 155.083 70.083) (end 155.083 69.2439) (width 0.4) (layer "F.Cu") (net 5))
 (segment (start 155.5 51) (end 159 47.5) (width 0.5) (layer "F.Cu") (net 5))
 (via (at 157 71.1273) (size 1.4) (drill 0.8) (layers "F.Cu" "B.Cu") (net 5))
 (segment (start 184 66.5) (end 184.249 66.749) (width 0.5) (layer "B.Cu") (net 5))
 (segment (start 182.5 66.5) (end 184 66.5) (width 0.5) (layer "B.Cu") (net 5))
 (segment (start 183.201 71.799) (end 183.6517 71.3483) (width 0.4) (layer "B.Cu") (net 5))
 (segment (start 157 71.1273) (end 157.6717 71.799) (width 0.4) (layer "B.Cu") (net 5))
 (segment (start 184.249 66.749) (end 184.249 70.751) (width 0.5) (layer "B.Cu") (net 5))
 (segment (start 184.249 70.751) (end 183.6517 71.3483) (width 0.5) (layer "B.Cu") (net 5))
 (segment (start 157.6717 71.799) (end 183.201 71.799) (width 0.4) (layer "B.Cu") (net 5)))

